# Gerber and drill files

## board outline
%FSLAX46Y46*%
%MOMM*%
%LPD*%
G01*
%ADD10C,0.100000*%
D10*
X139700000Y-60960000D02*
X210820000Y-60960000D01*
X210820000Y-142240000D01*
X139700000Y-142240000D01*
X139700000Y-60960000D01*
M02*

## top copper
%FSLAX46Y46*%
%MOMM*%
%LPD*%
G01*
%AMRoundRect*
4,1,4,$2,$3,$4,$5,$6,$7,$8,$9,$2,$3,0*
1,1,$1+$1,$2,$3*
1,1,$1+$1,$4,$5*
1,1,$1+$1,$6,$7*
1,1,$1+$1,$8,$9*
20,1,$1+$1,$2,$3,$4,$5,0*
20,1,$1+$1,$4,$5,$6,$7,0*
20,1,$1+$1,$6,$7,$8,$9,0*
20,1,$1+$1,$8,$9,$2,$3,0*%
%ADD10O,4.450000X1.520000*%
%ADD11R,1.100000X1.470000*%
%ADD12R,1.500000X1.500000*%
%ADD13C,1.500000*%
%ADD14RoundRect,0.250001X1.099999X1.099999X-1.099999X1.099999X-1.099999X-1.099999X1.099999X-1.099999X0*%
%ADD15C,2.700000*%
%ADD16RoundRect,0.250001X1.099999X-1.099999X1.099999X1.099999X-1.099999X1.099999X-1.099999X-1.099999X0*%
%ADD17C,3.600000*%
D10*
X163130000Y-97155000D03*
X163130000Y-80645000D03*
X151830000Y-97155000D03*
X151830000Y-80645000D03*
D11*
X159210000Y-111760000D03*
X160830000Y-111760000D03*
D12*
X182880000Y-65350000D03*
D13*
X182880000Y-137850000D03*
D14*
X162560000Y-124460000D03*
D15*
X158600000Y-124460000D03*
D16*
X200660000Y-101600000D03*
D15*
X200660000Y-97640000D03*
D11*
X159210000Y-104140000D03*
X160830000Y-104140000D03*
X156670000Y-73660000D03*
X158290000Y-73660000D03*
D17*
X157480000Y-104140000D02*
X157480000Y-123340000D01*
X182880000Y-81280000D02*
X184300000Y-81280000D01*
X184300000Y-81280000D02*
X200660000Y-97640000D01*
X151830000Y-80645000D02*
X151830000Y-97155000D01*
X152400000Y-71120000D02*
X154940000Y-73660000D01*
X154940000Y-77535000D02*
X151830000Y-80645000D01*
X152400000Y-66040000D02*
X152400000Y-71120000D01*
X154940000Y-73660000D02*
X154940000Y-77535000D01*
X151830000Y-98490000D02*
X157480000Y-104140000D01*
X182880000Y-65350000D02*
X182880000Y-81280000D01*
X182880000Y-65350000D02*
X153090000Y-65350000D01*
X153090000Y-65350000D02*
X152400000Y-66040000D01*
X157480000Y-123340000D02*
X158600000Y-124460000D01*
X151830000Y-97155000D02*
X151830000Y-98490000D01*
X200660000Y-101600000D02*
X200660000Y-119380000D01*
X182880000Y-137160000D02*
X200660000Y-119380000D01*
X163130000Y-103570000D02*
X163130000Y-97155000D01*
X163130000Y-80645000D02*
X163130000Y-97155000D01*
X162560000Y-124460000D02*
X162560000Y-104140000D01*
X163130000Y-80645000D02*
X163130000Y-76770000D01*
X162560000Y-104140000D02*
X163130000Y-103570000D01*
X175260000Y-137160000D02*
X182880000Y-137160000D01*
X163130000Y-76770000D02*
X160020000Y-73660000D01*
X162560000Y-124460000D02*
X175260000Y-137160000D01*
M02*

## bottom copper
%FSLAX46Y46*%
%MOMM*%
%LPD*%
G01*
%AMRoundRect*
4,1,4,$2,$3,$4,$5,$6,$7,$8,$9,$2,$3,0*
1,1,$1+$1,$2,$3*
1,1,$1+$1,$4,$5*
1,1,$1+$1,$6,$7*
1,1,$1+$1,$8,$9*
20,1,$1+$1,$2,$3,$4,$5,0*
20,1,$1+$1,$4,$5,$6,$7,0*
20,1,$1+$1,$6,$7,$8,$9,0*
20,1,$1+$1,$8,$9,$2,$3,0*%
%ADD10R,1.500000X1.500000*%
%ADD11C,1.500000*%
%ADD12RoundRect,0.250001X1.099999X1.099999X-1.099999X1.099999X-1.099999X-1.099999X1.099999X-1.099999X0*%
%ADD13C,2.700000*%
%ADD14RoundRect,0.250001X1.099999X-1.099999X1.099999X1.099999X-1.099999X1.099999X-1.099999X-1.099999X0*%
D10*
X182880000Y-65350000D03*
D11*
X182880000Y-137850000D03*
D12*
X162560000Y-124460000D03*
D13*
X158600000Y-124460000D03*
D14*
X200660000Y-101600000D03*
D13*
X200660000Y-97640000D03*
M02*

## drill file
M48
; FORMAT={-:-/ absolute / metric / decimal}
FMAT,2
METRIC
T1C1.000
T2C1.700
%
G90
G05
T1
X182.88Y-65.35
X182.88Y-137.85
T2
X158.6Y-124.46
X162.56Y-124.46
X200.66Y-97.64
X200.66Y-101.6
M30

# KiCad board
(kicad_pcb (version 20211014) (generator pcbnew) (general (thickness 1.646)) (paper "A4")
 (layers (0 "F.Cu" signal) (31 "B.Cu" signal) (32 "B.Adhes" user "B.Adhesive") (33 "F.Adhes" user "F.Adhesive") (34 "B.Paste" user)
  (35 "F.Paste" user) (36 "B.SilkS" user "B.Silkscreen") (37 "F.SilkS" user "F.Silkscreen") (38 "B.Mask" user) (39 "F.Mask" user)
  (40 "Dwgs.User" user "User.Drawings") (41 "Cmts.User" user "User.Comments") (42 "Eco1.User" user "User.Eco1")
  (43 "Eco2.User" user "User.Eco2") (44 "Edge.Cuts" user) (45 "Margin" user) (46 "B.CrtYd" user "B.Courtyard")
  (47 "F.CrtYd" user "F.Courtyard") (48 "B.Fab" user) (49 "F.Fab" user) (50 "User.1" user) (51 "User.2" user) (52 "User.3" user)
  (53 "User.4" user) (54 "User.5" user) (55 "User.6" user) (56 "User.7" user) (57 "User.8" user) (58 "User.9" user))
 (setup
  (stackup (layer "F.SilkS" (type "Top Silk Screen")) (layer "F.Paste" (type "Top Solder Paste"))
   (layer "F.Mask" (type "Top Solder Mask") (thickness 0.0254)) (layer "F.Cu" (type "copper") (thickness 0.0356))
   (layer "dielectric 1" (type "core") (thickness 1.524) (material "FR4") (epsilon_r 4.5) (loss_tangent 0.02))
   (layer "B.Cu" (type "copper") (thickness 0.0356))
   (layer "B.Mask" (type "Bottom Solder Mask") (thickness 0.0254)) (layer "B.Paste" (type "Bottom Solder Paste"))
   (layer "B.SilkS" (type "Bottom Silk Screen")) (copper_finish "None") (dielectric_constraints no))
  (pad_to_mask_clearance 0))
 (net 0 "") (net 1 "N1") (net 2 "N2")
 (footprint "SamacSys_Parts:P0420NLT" (layer "F.Cu") (at 157.48 88.9 180)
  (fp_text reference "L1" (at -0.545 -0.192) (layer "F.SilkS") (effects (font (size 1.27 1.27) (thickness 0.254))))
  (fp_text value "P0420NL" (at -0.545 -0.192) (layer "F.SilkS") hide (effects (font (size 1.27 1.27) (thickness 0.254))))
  (pad "1" smd oval locked (at -5.65 -8.255 270) (size 1.52 4.45) (layers "F.Cu" "F.Paste" "F.Mask") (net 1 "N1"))
  (pad "2" smd oval locked (at -5.65 8.255 270) (size 1.52 4.45) (layers "F.Cu" "F.Paste" "F.Mask") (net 1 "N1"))
  (pad "3" smd oval locked (at 5.65 -8.255 270) (size 1.52 4.45) (layers "F.Cu" "F.Paste" "F.Mask") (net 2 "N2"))
  (pad "4" smd oval locked (at 5.65 8.255 270) (size 1.52 4.45) (layers "F.Cu" "F.Paste" "F.Mask") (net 2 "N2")))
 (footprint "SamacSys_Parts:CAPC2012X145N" (layer "F.Cu") (at 160.02 111.76)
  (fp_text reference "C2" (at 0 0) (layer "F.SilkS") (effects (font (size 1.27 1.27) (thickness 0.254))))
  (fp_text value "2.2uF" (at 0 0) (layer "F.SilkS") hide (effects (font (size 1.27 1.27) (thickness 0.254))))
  (pad "1" smd rect locked (at -0.81 0) (size 1.1 1.47) (layers "F.Cu" "F.Paste" "F.Mask") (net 2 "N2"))
  (pad "2" smd rect locked (at 0.81 0) (size 1.1 1.47) (layers "F.Cu" "F.Paste" "F.Mask") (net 1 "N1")))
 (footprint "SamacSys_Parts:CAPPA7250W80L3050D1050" (layer "F.Cu") (at 182.88 65.35 -90)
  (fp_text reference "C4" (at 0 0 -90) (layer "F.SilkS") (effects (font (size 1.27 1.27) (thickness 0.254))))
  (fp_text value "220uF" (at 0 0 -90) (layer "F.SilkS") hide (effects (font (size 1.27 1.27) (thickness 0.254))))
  (pad "1" thru_hole rect locked (at 0 0 270) (size 1.5 1.5) (drill 1) (layers *.Cu *.Mask) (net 2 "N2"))
  (pad "2" thru_hole circle locked (at 72.5 0 270) (size 1.5 1.5) (drill 1) (layers *.Cu *.Mask) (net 1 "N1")))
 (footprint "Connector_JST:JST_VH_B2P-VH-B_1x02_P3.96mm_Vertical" (layer "F.Cu") (at 162.56 124.46 180)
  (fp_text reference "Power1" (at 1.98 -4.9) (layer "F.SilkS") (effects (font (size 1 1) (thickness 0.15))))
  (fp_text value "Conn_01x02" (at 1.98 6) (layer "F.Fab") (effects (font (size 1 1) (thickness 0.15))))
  (pad "1" thru_hole roundrect (at 0 0 180) (size 2.7 2.7) (drill 1.7) (layers *.Cu *.Mask) (roundrect_rratio 0.09259296296) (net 1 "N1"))
  (pad "2" thru_hole circle (at 3.96 0 180) (size 2.7 2.7) (drill 1.7) (layers *.Cu *.Mask) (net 2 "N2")))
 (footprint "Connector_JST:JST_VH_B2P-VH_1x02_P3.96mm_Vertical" (layer "F.Cu") (at 200.66 101.6 90)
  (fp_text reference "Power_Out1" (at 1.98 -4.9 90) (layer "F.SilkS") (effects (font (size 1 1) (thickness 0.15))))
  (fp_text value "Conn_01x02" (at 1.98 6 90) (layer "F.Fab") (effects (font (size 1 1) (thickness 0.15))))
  (pad "1" thru_hole roundrect (at 0 0 90) (size 2.7 2.7) (drill 1.7) (layers *.Cu *.Mask) (roundrect_rratio 0.09259296296) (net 1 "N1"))
  (pad "2" thru_hole circle (at 3.96 0 90) (size 2.7 2.7) (drill 1.7) (layers *.Cu *.Mask) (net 2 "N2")))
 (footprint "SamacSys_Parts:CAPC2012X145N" (layer "F.Cu") (at 160.02 104.14)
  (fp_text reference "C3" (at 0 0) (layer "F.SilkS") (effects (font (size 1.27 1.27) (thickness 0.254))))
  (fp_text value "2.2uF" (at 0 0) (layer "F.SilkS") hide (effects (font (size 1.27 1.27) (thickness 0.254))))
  (pad "1" smd rect locked (at -0.81 0) (size 1.1 1.47) (layers "F.Cu" "F.Paste" "F.Mask") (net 2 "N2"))
  (pad "2" smd rect locked (at 0.81 0) (size 1.1 1.47) (layers "F.Cu" "F.Paste" "F.Mask") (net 1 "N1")))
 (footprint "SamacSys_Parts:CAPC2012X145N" (layer "F.Cu") (at 157.48 73.66)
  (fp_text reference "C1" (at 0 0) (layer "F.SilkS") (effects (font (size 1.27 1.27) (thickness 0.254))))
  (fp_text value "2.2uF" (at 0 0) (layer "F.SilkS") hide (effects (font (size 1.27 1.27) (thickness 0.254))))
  (pad "1" smd rect locked (at -0.81 0) (size 1.1 1.47) (layers "F.Cu" "F.Paste" "F.Mask") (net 2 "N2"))
  (pad "2" smd rect locked (at 0.81 0) (size 1.1 1.47) (layers "F.Cu" "F.Paste" "F.Mask") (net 1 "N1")))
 (gr_rect (start 139.7 60.96) (end 210.82 142.24) (layer "Edge.Cuts") (width 0.1) (fill none))
 (segment (start 157.48 104.14) (end 157.48 123.34) (width 3.6) (layer "F.Cu") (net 2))
 (segment (start 182.88 81.28) (end 184.3 81.28) (width 3.6) (layer "F.Cu") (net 2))
 (segment (start 184.3 81.28) (end 200.66 97.64) (width 3.6) (layer "F.Cu") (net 2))
 (segment (start 151.83 80.645) (end 151.83 97.155) (width 3.6) (layer "F.Cu") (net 2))
 (segment (start 152.4 71.12) (end 154.94 73.66) (width 3.6) (layer "F.Cu") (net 2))
 (segment (start 154.94 77.535) (end 151.83 80.645) (width 3.6) (layer "F.Cu") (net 2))
 (segment (start 152.4 66.04) (end 152.4 71.12) (width 3.6) (layer "F.Cu") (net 2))
 (segment (start 154.94 73.66) (end 154.94 77.535) (width 3.6) (layer "F.Cu") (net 2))
 (segment (start 151.83 98.49) (end 157.48 104.14) (width 3.6) (layer "F.Cu") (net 2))
 (segment (start 182.88 65.35) (end 182.88 81.28) (width 3.6) (layer "F.Cu") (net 2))
 (segment (start 182.88 65.35) (end 153.09 65.35) (width 3.6) (layer "F.Cu") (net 2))
 (segment (start 153.09 65.35) (end 152.4 66.04) (width 3.6) (layer "F.Cu") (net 2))
 (segment (start 157.48 123.34) (end 158.6 124.46) (width 3.6) (layer "F.Cu") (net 2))
 (segment (start 151.83 97.155) (end 151.83 98.49) (width 3.6) (layer "F.Cu") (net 2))
 (segment (start 200.66 101.6) (end 200.66 119.38) (width 3.6) (layer "F.Cu") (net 1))
 (segment (start 182.88 137.16) (end 200.66 119.38) (width 3.6) (layer "F.Cu") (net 1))
 (segment (start 163.13 103.57) (end 163.13 97.155) (width 3.6) (layer "F.Cu") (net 1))
 (segment (start 163.13 80.645) (end 163.13 97.155) (width 3.6) (layer "F.Cu") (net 1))
 (segment (start 162.56 124.46) (end 162.56 104.14) (width 3.6) (layer "F.Cu") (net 1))
 (segment (start 163.13 80.645) (end 163.13 76.77) (width 3.6) (layer "F.Cu") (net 1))
 (segment (start 162.56 104.14) (end 163.13 103.57) (width 3.6) (layer "F.Cu") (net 1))
 (segment (start 175.26 137.16) (end 182.88 137.16) (width 3.6) (layer "F.Cu") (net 1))
 (segment (start 163.13 76.77) (end 160.02 73.66) (width 3.6) (layer "F.Cu") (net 1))
 (segment (start 162.56 124.46) (end 175.26 137.16) (width 3.6) (layer "F.Cu") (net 1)))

